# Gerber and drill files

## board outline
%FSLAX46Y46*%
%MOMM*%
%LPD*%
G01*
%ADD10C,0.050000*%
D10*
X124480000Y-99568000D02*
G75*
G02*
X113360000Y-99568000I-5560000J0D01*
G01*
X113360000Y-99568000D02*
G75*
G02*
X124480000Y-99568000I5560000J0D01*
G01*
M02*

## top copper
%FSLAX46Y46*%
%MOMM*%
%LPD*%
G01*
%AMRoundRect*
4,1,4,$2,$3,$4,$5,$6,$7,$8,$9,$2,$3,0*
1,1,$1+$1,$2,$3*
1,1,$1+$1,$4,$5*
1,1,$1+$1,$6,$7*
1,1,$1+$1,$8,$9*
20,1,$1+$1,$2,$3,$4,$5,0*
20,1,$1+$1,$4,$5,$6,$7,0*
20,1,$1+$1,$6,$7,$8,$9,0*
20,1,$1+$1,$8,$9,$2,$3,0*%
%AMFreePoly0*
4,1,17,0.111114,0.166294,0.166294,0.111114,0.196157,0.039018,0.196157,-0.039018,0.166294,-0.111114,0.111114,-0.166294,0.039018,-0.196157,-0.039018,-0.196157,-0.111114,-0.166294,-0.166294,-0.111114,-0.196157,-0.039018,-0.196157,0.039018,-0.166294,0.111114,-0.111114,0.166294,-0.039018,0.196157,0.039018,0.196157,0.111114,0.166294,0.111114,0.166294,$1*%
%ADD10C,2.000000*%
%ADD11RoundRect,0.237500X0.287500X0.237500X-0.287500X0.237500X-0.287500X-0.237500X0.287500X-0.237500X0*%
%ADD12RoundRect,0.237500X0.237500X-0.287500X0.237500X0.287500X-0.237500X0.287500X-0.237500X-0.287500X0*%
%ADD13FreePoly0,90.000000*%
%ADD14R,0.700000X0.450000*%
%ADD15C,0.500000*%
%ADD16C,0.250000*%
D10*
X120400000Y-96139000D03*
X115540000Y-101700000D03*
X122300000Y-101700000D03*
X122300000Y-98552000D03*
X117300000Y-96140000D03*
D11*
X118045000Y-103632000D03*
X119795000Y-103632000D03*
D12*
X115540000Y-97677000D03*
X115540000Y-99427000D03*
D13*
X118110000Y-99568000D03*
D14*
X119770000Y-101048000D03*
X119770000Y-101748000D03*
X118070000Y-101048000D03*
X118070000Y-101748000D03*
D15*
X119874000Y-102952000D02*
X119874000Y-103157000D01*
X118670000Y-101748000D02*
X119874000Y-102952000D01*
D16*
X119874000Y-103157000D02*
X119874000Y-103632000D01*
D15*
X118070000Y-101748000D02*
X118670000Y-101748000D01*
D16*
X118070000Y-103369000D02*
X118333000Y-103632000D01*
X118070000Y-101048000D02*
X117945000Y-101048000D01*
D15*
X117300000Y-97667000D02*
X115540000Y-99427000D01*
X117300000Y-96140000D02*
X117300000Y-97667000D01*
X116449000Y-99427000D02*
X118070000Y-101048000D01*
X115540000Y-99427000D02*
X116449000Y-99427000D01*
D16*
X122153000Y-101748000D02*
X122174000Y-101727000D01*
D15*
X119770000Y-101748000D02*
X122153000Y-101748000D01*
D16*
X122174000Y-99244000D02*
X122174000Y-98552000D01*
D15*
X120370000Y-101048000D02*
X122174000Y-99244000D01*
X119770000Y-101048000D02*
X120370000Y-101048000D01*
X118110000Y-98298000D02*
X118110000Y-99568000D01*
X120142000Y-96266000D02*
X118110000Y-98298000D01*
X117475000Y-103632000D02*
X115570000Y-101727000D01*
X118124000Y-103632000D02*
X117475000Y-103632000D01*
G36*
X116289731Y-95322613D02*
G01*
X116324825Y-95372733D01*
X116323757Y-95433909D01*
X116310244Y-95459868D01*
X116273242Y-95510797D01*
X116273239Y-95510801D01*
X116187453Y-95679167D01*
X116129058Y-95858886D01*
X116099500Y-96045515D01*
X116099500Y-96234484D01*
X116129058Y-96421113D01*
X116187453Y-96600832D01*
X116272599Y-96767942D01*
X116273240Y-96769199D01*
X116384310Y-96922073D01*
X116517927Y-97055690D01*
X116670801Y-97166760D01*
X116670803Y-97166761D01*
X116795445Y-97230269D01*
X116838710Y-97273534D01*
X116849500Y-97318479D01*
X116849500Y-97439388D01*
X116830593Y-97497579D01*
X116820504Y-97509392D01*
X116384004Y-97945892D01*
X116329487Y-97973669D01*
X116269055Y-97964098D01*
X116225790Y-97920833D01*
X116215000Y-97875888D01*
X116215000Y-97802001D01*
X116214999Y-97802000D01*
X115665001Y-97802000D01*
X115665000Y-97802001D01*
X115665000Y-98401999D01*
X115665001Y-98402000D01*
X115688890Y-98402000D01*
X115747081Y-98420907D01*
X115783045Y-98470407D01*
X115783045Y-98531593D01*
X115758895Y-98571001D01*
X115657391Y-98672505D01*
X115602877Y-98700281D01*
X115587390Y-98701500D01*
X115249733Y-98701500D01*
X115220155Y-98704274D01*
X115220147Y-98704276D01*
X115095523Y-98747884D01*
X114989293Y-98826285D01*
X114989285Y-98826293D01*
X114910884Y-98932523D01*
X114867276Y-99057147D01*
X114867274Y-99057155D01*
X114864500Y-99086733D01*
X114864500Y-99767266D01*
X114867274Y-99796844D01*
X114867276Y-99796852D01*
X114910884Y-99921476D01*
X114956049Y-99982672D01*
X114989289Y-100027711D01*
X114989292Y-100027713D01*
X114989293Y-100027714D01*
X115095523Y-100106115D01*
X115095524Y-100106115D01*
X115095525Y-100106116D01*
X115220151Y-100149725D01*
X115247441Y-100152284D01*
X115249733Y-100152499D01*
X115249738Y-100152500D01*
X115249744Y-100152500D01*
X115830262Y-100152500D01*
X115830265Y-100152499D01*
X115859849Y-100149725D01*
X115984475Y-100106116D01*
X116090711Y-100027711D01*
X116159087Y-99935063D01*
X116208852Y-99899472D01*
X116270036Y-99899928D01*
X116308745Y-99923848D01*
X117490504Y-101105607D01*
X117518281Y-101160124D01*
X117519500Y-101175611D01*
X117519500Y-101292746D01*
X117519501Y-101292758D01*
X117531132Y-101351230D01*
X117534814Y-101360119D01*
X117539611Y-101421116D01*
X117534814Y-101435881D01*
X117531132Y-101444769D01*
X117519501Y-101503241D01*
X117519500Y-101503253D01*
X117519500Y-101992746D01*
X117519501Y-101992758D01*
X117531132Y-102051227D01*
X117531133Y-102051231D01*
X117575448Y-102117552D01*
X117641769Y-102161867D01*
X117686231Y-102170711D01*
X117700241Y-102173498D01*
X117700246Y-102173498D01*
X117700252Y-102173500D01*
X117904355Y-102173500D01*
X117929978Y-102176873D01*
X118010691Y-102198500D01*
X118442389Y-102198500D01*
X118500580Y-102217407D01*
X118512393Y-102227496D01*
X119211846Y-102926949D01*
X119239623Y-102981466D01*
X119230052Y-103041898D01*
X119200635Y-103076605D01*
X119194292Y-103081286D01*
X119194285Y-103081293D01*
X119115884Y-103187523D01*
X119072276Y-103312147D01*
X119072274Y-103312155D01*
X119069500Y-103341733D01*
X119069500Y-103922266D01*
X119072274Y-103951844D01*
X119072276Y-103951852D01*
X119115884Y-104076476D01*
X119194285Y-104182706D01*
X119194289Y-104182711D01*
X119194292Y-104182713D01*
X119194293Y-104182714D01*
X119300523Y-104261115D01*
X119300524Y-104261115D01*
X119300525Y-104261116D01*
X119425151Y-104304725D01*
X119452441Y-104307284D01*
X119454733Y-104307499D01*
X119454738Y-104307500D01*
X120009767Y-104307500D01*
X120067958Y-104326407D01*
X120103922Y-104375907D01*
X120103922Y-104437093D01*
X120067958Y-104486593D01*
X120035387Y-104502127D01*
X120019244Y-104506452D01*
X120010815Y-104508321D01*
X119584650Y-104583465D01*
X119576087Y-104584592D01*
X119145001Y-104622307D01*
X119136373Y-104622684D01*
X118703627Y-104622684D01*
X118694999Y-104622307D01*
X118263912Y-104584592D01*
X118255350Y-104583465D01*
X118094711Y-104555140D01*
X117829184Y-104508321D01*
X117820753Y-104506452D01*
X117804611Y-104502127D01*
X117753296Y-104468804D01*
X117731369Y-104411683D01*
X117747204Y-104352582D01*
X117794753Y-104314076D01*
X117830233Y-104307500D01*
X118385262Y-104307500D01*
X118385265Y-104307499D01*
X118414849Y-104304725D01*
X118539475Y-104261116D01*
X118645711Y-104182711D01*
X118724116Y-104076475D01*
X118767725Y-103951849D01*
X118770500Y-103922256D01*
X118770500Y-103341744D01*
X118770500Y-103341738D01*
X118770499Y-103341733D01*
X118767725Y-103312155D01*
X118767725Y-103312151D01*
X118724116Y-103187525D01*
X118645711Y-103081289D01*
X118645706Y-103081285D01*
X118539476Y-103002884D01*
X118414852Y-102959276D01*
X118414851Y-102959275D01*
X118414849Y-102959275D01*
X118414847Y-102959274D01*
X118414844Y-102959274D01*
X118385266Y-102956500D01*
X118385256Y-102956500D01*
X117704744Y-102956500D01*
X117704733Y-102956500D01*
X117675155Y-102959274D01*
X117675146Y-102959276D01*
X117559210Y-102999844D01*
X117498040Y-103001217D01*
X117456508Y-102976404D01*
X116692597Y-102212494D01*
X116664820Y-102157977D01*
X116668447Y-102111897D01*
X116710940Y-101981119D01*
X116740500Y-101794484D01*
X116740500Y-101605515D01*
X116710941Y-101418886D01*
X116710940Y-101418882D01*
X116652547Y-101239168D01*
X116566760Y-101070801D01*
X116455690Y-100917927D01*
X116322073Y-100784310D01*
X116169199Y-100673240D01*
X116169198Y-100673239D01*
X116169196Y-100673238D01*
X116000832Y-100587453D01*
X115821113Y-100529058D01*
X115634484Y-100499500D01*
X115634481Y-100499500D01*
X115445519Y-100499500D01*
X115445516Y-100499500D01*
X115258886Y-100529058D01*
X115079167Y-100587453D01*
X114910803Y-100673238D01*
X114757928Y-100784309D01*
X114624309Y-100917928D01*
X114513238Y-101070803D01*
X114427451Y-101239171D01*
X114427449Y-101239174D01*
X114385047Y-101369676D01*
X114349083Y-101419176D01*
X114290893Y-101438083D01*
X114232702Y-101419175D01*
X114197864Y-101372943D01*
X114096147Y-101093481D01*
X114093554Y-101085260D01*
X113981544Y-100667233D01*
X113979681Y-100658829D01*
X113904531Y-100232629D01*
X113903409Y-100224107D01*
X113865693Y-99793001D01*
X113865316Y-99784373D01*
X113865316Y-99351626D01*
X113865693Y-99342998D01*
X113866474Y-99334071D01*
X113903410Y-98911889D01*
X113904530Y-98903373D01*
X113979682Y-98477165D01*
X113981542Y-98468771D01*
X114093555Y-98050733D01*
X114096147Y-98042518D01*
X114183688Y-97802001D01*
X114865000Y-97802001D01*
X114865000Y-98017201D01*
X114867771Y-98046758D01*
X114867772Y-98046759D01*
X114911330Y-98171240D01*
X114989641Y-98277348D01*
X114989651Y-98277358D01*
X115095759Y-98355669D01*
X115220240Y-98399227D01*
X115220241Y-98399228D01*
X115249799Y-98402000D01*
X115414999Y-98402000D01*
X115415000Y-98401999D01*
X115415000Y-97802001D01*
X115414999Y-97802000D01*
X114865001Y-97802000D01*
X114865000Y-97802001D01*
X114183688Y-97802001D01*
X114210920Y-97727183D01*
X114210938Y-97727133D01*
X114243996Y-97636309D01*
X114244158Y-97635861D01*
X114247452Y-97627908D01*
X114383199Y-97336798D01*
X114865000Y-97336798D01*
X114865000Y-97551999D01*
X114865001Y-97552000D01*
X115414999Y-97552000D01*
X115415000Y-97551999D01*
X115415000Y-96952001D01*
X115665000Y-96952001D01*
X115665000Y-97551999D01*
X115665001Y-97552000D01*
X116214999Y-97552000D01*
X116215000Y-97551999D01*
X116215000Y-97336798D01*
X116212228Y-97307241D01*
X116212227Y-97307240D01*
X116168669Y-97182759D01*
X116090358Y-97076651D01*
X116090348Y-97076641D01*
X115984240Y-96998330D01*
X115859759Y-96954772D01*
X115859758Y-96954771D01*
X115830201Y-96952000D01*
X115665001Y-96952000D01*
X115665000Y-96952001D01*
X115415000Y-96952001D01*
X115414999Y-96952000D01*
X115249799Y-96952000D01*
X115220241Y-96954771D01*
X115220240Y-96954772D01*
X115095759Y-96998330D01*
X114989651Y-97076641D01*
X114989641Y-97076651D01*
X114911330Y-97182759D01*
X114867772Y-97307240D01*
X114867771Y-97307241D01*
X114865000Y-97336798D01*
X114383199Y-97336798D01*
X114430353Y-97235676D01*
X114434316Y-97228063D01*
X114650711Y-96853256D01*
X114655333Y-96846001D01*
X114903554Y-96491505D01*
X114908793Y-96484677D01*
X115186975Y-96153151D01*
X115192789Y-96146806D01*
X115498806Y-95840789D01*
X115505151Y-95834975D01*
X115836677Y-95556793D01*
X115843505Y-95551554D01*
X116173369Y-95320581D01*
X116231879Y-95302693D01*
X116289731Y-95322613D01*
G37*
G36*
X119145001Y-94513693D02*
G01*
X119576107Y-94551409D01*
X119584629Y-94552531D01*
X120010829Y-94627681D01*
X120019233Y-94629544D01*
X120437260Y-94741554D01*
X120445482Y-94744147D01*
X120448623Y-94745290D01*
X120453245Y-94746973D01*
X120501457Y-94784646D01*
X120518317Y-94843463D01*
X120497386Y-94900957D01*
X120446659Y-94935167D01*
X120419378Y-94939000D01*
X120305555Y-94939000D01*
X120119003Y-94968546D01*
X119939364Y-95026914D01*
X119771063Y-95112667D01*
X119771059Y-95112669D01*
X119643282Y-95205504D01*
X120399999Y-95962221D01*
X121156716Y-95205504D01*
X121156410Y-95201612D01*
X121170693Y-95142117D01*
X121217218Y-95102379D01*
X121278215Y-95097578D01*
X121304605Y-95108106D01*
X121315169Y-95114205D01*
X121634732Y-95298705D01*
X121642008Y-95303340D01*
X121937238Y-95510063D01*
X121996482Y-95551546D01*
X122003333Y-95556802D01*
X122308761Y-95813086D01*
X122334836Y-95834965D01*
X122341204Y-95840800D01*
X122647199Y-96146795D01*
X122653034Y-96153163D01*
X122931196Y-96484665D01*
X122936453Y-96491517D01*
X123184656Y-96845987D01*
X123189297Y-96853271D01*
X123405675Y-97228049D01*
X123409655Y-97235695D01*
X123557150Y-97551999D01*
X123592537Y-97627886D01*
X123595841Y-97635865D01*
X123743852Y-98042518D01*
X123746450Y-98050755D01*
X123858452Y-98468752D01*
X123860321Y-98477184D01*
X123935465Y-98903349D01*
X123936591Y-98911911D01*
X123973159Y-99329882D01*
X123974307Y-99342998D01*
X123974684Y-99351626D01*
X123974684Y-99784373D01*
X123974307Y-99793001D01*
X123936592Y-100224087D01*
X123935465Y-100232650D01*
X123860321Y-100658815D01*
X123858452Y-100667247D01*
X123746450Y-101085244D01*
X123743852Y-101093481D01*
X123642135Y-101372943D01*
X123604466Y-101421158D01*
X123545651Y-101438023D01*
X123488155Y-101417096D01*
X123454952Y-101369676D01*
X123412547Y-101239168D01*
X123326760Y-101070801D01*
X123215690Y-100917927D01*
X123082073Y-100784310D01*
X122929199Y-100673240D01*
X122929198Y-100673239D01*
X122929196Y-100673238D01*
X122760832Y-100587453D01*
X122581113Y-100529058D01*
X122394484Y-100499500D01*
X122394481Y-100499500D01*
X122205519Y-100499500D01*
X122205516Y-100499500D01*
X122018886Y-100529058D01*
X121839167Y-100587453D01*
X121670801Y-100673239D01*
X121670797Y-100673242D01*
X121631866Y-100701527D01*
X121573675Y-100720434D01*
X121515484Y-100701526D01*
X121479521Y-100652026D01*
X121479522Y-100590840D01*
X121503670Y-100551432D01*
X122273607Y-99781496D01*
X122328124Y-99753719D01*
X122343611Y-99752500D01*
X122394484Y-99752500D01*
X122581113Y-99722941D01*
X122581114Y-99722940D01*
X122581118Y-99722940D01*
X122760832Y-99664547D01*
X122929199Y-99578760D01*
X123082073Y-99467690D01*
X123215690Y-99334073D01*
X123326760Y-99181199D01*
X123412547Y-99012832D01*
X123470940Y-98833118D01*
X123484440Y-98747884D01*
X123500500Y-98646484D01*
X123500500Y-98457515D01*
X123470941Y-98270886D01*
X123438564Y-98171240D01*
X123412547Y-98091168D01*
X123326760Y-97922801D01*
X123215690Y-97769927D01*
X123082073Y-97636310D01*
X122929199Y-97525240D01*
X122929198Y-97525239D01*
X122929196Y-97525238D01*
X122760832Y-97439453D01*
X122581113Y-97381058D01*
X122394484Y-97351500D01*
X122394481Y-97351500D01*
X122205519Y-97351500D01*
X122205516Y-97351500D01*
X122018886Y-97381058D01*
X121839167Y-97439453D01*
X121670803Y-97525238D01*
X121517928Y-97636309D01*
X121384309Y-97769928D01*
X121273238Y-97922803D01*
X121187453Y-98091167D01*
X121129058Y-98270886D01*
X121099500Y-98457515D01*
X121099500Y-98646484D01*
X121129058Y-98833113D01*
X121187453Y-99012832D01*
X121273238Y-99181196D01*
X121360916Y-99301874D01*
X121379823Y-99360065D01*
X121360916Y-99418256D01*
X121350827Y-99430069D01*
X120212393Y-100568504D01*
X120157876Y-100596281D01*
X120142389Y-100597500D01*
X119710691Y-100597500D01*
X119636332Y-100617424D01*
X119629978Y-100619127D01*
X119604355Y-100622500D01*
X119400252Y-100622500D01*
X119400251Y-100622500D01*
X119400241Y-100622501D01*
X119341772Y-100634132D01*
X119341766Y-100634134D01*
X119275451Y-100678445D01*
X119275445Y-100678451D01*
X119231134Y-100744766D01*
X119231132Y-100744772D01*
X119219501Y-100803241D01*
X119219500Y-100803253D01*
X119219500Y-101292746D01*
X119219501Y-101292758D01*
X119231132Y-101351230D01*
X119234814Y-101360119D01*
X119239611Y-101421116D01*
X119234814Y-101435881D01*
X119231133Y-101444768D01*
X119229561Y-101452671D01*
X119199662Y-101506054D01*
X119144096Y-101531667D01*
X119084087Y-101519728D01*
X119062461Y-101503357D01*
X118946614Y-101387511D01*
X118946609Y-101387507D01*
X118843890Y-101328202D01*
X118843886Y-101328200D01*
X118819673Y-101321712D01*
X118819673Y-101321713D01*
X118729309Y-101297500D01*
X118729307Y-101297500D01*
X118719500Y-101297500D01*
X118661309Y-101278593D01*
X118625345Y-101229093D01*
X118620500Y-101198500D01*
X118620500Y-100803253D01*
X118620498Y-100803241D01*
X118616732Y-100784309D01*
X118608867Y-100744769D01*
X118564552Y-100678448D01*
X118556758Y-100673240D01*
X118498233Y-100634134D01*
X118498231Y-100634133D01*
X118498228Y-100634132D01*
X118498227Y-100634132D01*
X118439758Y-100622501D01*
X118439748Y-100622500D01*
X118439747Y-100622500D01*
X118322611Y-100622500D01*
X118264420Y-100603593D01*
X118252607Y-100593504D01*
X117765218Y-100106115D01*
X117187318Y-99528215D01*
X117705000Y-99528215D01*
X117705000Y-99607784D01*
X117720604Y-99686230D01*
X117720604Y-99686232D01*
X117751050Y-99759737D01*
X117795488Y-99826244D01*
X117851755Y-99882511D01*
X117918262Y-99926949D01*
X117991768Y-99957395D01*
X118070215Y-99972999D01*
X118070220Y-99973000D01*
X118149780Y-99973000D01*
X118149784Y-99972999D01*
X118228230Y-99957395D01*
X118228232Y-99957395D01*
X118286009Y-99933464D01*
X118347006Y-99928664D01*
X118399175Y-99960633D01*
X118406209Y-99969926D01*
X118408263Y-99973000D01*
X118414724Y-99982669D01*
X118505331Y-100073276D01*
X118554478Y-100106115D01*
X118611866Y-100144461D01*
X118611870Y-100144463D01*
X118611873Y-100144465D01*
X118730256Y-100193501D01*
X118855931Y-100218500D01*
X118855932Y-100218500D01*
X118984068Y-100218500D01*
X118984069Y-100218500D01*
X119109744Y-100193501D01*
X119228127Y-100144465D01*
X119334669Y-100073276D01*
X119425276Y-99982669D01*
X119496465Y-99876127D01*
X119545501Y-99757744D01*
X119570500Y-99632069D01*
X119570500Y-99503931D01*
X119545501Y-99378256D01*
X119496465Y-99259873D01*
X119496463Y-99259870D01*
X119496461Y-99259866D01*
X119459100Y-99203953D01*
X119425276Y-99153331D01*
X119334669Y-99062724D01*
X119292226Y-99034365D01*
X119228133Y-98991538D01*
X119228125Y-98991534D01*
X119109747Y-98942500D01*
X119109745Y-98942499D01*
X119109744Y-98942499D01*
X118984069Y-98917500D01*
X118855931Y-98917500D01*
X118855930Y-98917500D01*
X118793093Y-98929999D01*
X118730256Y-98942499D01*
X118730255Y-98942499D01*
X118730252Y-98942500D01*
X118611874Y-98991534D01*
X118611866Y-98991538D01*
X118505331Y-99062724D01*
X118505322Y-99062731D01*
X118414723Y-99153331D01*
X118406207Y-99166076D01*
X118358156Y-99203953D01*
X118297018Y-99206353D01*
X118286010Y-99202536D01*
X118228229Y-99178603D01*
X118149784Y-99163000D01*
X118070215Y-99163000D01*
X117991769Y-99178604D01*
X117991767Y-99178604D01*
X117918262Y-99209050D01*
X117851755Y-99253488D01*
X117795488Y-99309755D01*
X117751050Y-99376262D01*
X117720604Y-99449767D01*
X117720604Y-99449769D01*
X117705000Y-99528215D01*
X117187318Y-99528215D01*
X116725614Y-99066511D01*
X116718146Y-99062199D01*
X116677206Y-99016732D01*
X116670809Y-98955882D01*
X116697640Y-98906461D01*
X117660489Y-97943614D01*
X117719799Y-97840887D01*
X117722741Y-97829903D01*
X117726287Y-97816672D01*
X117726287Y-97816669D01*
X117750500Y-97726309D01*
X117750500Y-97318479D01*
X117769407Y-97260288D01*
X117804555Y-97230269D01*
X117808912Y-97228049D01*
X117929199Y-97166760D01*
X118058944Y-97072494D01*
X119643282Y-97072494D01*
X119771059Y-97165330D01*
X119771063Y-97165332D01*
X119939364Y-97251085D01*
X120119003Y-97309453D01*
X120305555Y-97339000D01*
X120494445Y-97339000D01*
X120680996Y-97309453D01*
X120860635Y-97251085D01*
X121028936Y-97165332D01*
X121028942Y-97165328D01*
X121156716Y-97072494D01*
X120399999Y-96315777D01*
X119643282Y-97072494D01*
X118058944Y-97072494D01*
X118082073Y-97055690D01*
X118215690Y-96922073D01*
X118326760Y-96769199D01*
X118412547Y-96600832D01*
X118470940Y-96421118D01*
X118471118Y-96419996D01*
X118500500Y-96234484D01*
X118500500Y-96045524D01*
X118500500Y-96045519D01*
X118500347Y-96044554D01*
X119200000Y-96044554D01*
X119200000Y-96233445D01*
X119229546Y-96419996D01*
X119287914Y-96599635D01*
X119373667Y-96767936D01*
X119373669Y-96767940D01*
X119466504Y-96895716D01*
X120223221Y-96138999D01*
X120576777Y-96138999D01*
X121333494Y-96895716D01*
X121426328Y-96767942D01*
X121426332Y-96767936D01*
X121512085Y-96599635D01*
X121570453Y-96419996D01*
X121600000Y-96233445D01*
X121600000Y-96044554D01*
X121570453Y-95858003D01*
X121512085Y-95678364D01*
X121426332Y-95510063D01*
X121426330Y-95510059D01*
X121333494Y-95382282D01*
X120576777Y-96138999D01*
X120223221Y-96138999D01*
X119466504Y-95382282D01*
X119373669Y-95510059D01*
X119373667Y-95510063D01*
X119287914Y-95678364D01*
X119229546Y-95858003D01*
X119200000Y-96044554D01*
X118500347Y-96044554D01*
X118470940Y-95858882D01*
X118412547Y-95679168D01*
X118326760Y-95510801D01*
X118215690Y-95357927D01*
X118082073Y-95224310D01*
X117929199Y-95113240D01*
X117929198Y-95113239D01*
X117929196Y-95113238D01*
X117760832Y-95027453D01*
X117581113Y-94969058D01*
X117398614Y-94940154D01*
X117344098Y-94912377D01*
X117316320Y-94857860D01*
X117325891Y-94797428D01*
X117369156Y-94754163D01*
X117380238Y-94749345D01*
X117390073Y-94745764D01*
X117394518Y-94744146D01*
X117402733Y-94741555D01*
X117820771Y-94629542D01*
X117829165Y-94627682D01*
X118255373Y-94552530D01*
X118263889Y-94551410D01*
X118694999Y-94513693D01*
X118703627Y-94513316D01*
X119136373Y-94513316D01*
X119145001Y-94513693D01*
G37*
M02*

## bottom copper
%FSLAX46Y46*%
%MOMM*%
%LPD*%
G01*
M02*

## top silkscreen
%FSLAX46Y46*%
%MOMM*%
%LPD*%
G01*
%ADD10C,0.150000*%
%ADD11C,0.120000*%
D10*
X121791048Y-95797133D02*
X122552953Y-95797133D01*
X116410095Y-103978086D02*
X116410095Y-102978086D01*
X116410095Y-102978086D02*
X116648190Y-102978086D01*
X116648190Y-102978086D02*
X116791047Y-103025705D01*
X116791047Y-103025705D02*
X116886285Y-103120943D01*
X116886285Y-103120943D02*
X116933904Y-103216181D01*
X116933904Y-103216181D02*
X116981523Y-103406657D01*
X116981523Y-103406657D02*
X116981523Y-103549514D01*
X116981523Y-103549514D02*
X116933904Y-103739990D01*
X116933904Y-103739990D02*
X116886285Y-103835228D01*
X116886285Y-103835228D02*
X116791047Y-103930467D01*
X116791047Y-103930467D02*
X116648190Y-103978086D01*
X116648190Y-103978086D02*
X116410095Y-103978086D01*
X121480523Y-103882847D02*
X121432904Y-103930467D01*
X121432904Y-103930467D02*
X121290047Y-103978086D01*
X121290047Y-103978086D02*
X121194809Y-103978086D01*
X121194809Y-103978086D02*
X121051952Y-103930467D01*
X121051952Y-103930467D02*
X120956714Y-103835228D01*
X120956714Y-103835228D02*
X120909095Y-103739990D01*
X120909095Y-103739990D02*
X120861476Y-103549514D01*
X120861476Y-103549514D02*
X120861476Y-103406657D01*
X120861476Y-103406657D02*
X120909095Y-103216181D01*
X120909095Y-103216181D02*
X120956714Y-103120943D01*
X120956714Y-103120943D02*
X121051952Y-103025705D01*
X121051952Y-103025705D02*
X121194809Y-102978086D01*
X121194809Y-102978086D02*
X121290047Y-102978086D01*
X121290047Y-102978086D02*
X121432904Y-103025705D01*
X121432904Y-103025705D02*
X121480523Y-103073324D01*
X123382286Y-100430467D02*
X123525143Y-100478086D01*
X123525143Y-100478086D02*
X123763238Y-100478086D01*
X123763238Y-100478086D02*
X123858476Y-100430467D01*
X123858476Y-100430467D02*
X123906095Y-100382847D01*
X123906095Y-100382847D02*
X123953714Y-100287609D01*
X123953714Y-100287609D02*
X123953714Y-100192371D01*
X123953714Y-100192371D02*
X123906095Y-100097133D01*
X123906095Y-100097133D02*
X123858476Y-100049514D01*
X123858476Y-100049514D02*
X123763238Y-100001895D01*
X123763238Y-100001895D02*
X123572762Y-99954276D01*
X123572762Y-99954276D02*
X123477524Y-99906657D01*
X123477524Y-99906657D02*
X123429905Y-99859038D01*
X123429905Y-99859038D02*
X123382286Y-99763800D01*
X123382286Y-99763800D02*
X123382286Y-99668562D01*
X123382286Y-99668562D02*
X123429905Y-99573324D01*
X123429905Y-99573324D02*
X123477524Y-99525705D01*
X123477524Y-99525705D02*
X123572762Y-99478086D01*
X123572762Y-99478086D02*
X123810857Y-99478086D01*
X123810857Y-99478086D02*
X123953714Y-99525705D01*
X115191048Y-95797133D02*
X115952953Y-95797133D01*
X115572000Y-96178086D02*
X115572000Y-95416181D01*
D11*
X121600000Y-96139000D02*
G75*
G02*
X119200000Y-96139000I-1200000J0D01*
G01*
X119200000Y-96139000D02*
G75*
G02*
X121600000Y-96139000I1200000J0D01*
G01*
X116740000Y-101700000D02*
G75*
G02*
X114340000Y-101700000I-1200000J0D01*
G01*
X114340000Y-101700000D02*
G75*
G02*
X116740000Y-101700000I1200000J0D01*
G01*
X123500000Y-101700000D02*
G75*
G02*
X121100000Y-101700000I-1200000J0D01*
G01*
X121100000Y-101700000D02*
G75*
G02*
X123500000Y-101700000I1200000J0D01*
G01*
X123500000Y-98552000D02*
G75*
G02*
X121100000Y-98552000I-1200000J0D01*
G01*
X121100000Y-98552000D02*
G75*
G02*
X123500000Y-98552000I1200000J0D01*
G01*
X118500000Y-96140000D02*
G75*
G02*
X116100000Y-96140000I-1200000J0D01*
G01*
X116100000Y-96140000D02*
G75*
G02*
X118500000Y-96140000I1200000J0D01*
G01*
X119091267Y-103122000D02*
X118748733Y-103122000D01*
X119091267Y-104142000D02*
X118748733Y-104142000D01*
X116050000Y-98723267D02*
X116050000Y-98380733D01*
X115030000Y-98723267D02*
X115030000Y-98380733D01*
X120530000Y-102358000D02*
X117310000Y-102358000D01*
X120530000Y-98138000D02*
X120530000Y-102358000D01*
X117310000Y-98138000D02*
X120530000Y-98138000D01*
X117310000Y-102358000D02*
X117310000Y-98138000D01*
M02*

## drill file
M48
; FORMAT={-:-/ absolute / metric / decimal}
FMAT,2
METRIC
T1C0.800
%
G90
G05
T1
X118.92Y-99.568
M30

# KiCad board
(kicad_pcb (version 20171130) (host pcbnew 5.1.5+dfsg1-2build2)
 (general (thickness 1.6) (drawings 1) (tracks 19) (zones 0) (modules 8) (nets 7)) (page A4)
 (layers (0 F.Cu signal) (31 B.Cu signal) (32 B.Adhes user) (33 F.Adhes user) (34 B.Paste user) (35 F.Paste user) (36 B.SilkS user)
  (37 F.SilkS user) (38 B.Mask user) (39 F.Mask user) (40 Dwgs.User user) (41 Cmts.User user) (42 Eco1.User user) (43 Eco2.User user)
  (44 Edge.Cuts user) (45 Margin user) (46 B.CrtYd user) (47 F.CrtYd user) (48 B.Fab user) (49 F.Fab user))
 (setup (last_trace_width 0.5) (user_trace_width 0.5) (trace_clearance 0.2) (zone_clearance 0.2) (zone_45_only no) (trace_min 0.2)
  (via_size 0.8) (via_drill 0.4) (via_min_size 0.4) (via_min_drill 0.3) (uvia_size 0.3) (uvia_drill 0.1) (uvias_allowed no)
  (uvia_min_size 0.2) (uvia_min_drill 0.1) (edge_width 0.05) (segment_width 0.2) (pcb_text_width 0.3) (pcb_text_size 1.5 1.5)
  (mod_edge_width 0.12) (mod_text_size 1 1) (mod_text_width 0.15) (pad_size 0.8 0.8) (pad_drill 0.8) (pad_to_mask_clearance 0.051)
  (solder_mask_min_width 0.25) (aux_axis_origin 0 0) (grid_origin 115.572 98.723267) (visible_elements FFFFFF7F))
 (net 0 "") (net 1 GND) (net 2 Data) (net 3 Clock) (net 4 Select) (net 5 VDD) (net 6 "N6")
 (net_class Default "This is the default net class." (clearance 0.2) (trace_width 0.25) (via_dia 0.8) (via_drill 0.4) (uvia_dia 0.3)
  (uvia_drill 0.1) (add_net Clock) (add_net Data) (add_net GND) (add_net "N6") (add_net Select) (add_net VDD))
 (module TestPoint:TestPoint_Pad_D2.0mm (layer F.Cu) (at 120.4 96.139)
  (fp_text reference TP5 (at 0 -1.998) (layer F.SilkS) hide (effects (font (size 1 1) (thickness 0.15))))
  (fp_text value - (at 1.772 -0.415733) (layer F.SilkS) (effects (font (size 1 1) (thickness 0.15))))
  (fp_circle (center 0 0) (end 0 1.2) (layer F.SilkS) (width 0.12))
  (pad 1 smd circle (at 0 0) (size 2 2) (layers F.Cu F.Mask) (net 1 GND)))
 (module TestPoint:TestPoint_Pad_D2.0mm (layer F.Cu) (at 115.54 101.7)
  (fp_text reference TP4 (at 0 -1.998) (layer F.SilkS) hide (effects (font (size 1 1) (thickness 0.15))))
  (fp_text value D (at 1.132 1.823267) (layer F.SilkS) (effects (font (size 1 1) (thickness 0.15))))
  (fp_circle (center 0 0) (end 0 1.2) (layer F.SilkS) (width 0.12))
  (pad 1 smd circle (at 0 0) (size 2 2) (layers F.Cu F.Mask) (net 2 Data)))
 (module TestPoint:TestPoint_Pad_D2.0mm (layer F.Cu) (at 122.3 101.7)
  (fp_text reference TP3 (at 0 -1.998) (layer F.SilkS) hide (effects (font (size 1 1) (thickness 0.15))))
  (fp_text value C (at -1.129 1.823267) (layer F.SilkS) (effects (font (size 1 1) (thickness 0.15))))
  (fp_circle (center 0 0) (end 0 1.2) (layer F.SilkS) (width 0.12))
  (pad 1 smd circle (at 0 0) (size 2 2) (layers F.Cu F.Mask) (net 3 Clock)))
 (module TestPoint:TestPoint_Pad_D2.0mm (layer F.Cu) (at 122.3 98.552)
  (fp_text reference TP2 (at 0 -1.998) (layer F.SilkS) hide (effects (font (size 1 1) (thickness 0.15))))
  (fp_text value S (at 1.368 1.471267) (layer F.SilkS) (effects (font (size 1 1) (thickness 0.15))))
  (fp_circle (center 0 0) (end 0 1.2) (layer F.SilkS) (width 0.12))
  (pad 1 smd circle (at 0 0) (size 2 2) (layers F.Cu F.Mask) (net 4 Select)))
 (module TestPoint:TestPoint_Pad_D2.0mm (layer F.Cu) (at 117.3 96.14)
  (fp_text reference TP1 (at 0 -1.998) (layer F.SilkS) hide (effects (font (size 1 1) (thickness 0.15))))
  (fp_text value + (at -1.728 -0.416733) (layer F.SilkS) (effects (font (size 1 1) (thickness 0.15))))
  (fp_circle (center 0 0) (end 0 1.2) (layer F.SilkS) (width 0.12))
  (pad 1 smd circle (at 0 0) (size 2 2) (layers F.Cu F.Mask) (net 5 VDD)))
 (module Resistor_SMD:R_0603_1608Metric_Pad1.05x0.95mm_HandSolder (layer F.Cu) (at 118.92 103.632 180)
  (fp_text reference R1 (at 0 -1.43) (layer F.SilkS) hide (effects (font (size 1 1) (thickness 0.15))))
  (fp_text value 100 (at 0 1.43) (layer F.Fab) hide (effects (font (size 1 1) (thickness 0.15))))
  (fp_line (start -0.171267 0.51) (end 0.171267 0.51) (layer F.SilkS) (width 0.12))
  (fp_line (start -0.171267 -0.51) (end 0.171267 -0.51) (layer F.SilkS) (width 0.12))
  (pad 2 smd roundrect (at 0.875 0 180) (size 1.05 0.95) (layers F.Cu F.Paste F.Mask) (roundrect_rratio 0.25) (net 2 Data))
  (pad 1 smd roundrect (at -0.875 0 180) (size 1.05 0.95) (layers F.Cu F.Paste F.Mask) (roundrect_rratio 0.25) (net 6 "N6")))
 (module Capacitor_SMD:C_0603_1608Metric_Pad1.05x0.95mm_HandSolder (layer F.Cu) (at 115.54 98.552 90)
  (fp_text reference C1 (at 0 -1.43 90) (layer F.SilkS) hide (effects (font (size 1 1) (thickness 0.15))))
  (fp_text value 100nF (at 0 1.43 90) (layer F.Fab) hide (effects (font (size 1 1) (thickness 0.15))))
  (fp_line (start -0.171267 0.51) (end 0.171267 0.51) (layer F.SilkS) (width 0.12))
  (fp_line (start -0.171267 -0.51) (end 0.171267 -0.51) (layer F.SilkS) (width 0.12))
  (pad 2 smd roundrect (at 0.875 0 90) (size 1.05 0.95) (layers F.Cu F.Paste F.Mask) (roundrect_rratio 0.25) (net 1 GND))
  (pad 1 smd roundrect (at -0.875 0 90) (size 1.05 0.95) (layers F.Cu F.Paste F.Mask) (roundrect_rratio 0.25) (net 5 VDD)))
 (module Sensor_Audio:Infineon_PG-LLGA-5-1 (layer F.Cu) (at 118.92 100.248 90)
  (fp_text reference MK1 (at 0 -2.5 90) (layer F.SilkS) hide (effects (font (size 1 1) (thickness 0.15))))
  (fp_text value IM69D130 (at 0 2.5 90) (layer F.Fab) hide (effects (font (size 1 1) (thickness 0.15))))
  (fp_line (start -2.11 1.61) (end -2.11 -1.61) (layer F.SilkS) (width 0.12))
  (fp_line (start 2.11 1.61) (end -2.11 1.61) (layer F.SilkS) (width 0.12))
  (fp_line (start 2.11 -1.61) (end 2.11 1.61) (layer F.SilkS) (width 0.12))
  (fp_line (start -2.11 -1.61) (end 2.11 -1.61) (layer F.SilkS) (width 0.12))
  (pad 5 smd custom (at 0.68 -0.81 90) (size 0.4 0.4) (layers F.Cu F.Mask) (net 1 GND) (zone_connect 0)
   (options (clearance outline) (anchor circle)) (primitives))
  (pad "" smd custom (at 1.08 -0.693 90) (size 0.3 0.3) (layers F.Paste) (zone_connect 0) (options (clearance outline) (anchor circle))
   (primitives))
  (pad "" smd custom (at 0.28 -0.693 90) (size 0.3 0.3) (layers F.Paste) (zone_connect 0) (options (clearance outline) (anchor circle))
   (primitives))
  (pad "" smd custom (at -0.12 0 90) (size 0.3 0.3) (layers F.Paste) (zone_connect 0) (options (clearance outline) (anchor circle))
   (primitives))
  (pad "" smd custom (at 0.28 0.693 90) (size 0.3 0.3) (layers F.Paste) (zone_connect 0) (options (clearance outline) (anchor circle))
   (primitives))
  (pad "" smd custom (at 1.08 0.693 90) (size 0.3 0.3) (layers F.Paste) (zone_connect 0) (options (clearance outline) (anchor circle))
   (primitives))
  (pad "" smd custom (at 1.48 0 90) (size 0.3 0.3) (layers F.Paste) (zone_connect 0) (options (clearance outline) (anchor circle))
   (primitives))
  (pad "" smd custom (at -0.8 0.725 90) (size 0.3 0.3) (layers F.Paste) (zone_connect 0) (options (clearance outline) (anchor circle))
   (primitives))
  (pad "" smd custom (at -1.5 0.725 90) (size 0.3 0.3) (layers F.Paste) (zone_connect 0) (options (clearance outline) (anchor circle))
   (primitives))
  (pad "" smd custom (at -0.8 -0.725 90) (size 0.3 0.3) (layers F.Paste) (zone_connect 0) (options (clearance outline) (anchor circle))
   (primitives))
  (pad "" smd custom (at -1.5 -0.725 90) (size 0.3 0.3) (layers F.Paste) (zone_connect 0) (options (clearance outline) (anchor circle))
   (primitives))
  (pad "" np_thru_hole circle (at 0.68 0 90) (size 0.8 0.8) (drill 0.8) (layers *.Cu *.Mask))
  (pad 4 smd rect (at -0.8 0.85 90) (size 0.45 0.7) (layers F.Cu F.Mask) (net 4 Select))
  (pad 3 smd rect (at -1.5 0.85 90) (size 0.45 0.7) (layers F.Cu F.Mask) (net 3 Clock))
  (pad 2 smd rect (at -0.8 -0.85 90) (size 0.45 0.7) (layers F.Cu F.Mask) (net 5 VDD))
  (pad 1 smd rect (at -1.5 -0.85 90) (size 0.45 0.7) (layers F.Cu F.Mask) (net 6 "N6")))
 (gr_circle (center 118.92 99.568) (end 124.48 99.568) (layer Edge.Cuts) (width 0.05))
 (segment (start 119.874 102.952) (end 119.874 103.157) (width 0.5) (layer F.Cu) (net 6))
 (segment (start 118.67 101.748) (end 119.874 102.952) (width 0.5) (layer F.Cu) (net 6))
 (segment (start 119.874 103.157) (end 119.874 103.632) (width 0.25) (layer F.Cu) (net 6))
 (segment (start 118.07 101.748) (end 118.67 101.748) (width 0.5) (layer F.Cu) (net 6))
 (segment (start 118.07 103.369) (end 118.333 103.632) (width 0.25) (layer F.Cu) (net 2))
 (segment (start 118.07 101.048) (end 117.945 101.048) (width 0.25) (layer F.Cu) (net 5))
 (segment (start 117.3 97.667) (end 115.54 99.427) (width 0.5) (layer F.Cu) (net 5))
 (segment (start 117.3 96.14) (end 117.3 97.667) (width 0.5) (layer F.Cu) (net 5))
 (segment (start 116.449 99.427) (end 118.07 101.048) (width 0.5) (layer F.Cu) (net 5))
 (segment (start 115.54 99.427) (end 116.449 99.427) (width 0.5) (layer F.Cu) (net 5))
 (segment (start 122.153 101.748) (end 122.174 101.727) (width 0.25) (layer F.Cu) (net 3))
 (segment (start 119.77 101.748) (end 122.153 101.748) (width 0.5) (layer F.Cu) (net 3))
 (segment (start 122.174 99.244) (end 122.174 98.552) (width 0.25) (layer F.Cu) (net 4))
 (segment (start 120.37 101.048) (end 122.174 99.244) (width 0.5) (layer F.Cu) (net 4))
 (segment (start 119.77 101.048) (end 120.37 101.048) (width 0.5) (layer F.Cu) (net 4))
 (segment (start 118.11 98.298) (end 118.11 99.568) (width 0.5) (layer F.Cu) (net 1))
 (segment (start 120.142 96.266) (end 118.11 98.298) (width 0.5) (layer F.Cu) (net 1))
 (segment (start 117.475 103.632) (end 115.57 101.727) (width 0.5) (layer F.Cu) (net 2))
 (segment (start 118.124 103.632) (end 117.475 103.632) (width 0.5) (layer F.Cu) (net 2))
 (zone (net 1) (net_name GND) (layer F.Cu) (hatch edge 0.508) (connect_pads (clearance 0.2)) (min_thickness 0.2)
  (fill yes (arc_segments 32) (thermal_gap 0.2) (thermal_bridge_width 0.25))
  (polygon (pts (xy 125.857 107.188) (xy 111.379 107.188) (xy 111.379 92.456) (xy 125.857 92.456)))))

